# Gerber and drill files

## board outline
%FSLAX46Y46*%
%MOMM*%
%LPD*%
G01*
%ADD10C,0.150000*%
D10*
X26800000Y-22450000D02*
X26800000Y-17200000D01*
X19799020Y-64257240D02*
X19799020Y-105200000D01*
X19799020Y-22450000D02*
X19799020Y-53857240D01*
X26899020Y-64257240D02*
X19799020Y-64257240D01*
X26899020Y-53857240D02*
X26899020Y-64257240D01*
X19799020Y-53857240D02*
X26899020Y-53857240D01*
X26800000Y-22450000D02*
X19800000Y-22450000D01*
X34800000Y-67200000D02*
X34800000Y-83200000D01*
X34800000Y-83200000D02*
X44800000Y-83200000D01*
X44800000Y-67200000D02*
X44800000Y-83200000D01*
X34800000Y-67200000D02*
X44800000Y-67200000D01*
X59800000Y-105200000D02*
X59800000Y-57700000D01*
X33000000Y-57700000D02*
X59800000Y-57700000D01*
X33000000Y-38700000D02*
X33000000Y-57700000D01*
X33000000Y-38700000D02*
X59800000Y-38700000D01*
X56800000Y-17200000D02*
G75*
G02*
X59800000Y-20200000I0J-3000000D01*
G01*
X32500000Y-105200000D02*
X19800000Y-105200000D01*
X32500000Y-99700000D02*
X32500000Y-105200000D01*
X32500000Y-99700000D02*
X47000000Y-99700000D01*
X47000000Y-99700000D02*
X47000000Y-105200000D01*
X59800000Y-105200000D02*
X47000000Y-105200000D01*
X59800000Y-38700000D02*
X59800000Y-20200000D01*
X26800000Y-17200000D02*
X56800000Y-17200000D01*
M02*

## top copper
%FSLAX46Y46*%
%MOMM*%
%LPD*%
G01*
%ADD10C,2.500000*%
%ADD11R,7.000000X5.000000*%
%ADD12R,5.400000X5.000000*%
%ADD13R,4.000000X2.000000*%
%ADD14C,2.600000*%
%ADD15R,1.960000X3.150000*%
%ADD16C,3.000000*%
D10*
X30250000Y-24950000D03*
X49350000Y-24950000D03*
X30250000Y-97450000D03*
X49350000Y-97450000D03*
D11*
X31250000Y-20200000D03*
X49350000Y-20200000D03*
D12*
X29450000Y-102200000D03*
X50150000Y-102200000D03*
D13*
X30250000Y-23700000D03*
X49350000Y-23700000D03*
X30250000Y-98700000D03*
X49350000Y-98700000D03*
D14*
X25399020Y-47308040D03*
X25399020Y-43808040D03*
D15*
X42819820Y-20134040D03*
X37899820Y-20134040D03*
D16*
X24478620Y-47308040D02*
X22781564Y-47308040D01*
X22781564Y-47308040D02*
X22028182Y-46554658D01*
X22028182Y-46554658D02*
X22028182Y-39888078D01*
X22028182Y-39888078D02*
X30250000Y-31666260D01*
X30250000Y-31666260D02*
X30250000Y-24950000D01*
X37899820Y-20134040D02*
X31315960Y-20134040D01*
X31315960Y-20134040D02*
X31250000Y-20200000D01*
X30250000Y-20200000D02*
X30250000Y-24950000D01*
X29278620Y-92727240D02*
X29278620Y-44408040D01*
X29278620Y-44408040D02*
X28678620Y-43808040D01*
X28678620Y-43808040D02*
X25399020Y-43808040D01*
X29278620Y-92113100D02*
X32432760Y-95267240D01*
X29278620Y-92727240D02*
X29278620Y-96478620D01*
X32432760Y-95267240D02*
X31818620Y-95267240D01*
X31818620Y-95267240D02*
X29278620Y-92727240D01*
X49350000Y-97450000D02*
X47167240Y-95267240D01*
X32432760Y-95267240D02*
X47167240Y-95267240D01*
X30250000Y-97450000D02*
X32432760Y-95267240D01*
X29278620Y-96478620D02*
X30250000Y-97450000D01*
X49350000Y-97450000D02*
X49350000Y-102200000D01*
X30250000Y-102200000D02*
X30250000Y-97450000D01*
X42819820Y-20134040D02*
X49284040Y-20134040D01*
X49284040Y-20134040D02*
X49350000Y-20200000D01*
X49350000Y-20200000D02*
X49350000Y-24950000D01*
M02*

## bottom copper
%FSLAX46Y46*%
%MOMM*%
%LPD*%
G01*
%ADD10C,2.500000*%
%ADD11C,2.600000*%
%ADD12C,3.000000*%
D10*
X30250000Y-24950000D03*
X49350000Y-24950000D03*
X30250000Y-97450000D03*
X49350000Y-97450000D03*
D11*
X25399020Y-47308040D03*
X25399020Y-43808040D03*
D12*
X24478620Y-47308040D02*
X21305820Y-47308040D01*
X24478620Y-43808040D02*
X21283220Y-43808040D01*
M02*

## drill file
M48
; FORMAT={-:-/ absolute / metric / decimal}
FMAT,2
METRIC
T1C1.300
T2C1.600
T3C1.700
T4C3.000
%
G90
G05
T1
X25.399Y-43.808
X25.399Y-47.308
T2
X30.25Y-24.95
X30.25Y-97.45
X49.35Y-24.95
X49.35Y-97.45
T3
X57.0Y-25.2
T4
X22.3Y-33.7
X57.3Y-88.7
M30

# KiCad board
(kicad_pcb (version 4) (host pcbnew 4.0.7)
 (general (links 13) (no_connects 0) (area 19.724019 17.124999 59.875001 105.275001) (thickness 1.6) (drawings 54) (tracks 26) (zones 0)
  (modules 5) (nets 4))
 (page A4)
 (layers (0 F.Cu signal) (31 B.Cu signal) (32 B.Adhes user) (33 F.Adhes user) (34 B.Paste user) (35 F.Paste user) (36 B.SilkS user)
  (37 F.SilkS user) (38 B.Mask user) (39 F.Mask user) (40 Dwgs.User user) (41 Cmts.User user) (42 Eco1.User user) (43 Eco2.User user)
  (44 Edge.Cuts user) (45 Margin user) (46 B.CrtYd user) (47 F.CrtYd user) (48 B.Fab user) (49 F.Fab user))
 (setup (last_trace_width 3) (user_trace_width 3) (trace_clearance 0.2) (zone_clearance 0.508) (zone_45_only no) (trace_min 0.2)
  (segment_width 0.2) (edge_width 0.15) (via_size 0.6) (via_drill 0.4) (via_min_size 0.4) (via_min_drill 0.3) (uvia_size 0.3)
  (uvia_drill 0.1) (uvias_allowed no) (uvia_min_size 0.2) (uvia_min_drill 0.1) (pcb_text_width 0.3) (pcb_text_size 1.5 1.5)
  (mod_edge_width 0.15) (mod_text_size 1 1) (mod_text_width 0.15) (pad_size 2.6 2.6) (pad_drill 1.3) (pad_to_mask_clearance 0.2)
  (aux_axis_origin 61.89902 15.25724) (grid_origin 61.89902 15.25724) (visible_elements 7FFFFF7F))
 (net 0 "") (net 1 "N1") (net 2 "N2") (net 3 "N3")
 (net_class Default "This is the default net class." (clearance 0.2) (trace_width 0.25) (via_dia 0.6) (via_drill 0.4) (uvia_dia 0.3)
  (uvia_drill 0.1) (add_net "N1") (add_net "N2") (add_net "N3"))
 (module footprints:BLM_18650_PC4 (layer F.Cu) (at 39.8 61.2)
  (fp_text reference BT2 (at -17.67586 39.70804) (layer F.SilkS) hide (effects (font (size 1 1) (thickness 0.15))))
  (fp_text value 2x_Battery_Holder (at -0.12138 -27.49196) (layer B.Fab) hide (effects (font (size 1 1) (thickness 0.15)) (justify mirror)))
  (pad 1 thru_hole circle (at -9.55 -36.25) (size 2.5 2.5) (drill 1.6) (layers *.Cu *.Mask) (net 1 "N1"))
  (pad 2 thru_hole circle (at 9.55 -36.25) (size 2.5 2.5) (drill 1.6) (layers *.Cu *.Mask) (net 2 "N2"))
  (pad 3 thru_hole circle (at -9.55 36.25) (size 2.5 2.5) (drill 1.6) (layers *.Cu *.Mask) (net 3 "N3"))
  (pad 4 thru_hole circle (at 9.55 36.25) (size 2.5 2.5) (drill 1.6) (layers *.Cu *.Mask) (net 3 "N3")))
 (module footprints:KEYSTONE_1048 (layer F.Cu) (at 39.8 61.2)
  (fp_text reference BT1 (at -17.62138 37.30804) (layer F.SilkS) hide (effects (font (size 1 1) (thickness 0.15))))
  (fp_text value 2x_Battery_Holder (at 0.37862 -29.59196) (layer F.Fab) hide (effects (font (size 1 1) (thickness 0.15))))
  (pad 1 smd rect (at -8.55 -41) (size 7 5) (layers F.Cu F.Paste F.Mask) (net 1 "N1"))
  (pad 2 smd rect (at 9.55 -41) (size 7 5) (layers F.Cu F.Paste F.Mask) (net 2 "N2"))
  (pad 3 smd rect (at -10.35 41) (size 5.4 5) (layers F.Cu F.Paste F.Mask) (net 3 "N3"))
  (pad 4 smd rect (at 10.35 41) (size 5.4 5) (layers F.Cu F.Paste F.Mask) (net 3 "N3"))
  (pad "" np_thru_hole circle (at 17.2 -36) (size 1.7 1.7) (drill 1.7) (layers *.Cu *.Mask))
  (pad "" np_thru_hole circle (at -17.5 -27.5) (size 3 3) (drill 3) (layers *.Cu *.Mask))
  (pad "" np_thru_hole circle (at 17.5 27.5) (size 3 3) (drill 3) (layers *.Cu *.Mask))
  (pad 1 smd rect (at -9.55 -37.5) (size 4 2) (layers F.Cu F.Paste F.Mask) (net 1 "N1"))
  (pad 2 smd rect (at 9.55 -37.5) (size 4 2) (layers F.Cu F.Paste F.Mask) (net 2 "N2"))
  (pad 3 smd rect (at -9.55 37.5) (size 4 2) (layers F.Cu F.Paste F.Mask) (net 3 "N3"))
  (pad 4 smd rect (at 9.55 37.5) (size 4 2) (layers F.Cu F.Paste F.Mask) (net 3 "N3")))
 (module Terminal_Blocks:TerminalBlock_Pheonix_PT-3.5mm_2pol (layer F.Cu) (at 25.39902 43.80804 270)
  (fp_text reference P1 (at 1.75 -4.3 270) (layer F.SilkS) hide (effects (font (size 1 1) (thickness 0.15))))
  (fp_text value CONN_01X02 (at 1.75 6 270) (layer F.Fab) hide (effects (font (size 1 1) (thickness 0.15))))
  (pad 2 thru_hole circle (at 3.5 0 270) (size 2.6 2.6) (drill 1.3) (layers *.Cu *.Mask) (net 1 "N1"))
  (pad 1 thru_hole circle (at 0 0 270) (size 2.6 2.6) (drill 1.3) (layers *.Cu *.Mask) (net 3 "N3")))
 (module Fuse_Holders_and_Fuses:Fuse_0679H (layer F.Cu) (at 40.35982 20.13404)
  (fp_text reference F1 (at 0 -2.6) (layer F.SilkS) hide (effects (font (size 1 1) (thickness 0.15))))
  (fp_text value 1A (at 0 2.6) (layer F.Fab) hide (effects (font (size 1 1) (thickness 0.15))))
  (pad 2 smd rect (at 2.46 0) (size 1.96 3.15) (layers F.Cu F.Paste F.Mask) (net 2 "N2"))
  (pad 1 smd rect (at -2.46 0) (size 1.96 3.15) (layers F.Cu F.Paste F.Mask) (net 1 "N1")))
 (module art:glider (layer F.Cu) (at 30.39902 37.75724)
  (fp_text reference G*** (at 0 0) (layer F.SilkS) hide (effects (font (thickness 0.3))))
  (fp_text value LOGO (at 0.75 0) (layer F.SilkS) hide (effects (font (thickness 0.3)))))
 (gr_line (start 26.8 22.45) (end 26.8 17.2) (layer Edge.Cuts) (width 0.15))
 (gr_line (start 19.79902 64.25724) (end 19.79902 105.2) (layer Edge.Cuts) (width 0.15))
 (gr_line (start 19.79902 22.45) (end 19.79902 53.85724) (layer Edge.Cuts) (width 0.15))
 (gr_line (start 26.89902 64.25724) (end 19.79902 64.25724) (layer Edge.Cuts) (width 0.15))
 (gr_line (start 26.89902 53.85724) (end 26.89902 64.25724) (layer Edge.Cuts) (width 0.15))
 (gr_line (start 19.79902 53.85724) (end 26.89902 53.85724) (layer Edge.Cuts) (width 0.15))
 (gr_line (start 26.8 22.45) (end 19.8 22.45) (layer Edge.Cuts) (width 0.15))
 (gr_line (start 34.8 67.2) (end 34.8 83.2) (layer Edge.Cuts) (width 0.15))
 (gr_line (start 34.8 83.2) (end 44.8 83.2) (layer Edge.Cuts) (width 0.15))
 (gr_line (start 44.8 67.2) (end 44.8 83.2) (layer Edge.Cuts) (width 0.15))
 (gr_line (start 34.8 67.2) (end 44.8 67.2) (layer Edge.Cuts) (width 0.15))
 (gr_line (start 59.8 105.2) (end 59.8 57.7) (layer Edge.Cuts) (width 0.15))
 (gr_line (start 33 57.7) (end 59.8 57.7) (layer Edge.Cuts) (width 0.15))
 (gr_line (start 33 38.7) (end 33 57.7) (layer Edge.Cuts) (width 0.15))
 (gr_line (start 33 38.7) (end 59.8 38.7) (layer Edge.Cuts) (width 0.15))
 (gr_arc (start 56.8 20.2) (end 56.8 17.2) (angle 90) (layer Edge.Cuts) (width 0.15))
 (gr_line (start 32.5 105.2) (end 19.8 105.2) (layer Edge.Cuts) (width 0.15))
 (gr_line (start 32.5 99.7) (end 32.5 105.2) (layer Edge.Cuts) (width 0.15))
 (gr_line (start 32.5 99.7) (end 47 99.7) (layer Edge.Cuts) (width 0.15))
 (gr_line (start 47 99.7) (end 47 105.2) (layer Edge.Cuts) (width 0.15))
 (gr_line (start 59.8 105.2) (end 47 105.2) (layer Edge.Cuts) (width 0.15))
 (gr_line (start 59.8 38.7) (end 59.8 20.2) (layer Edge.Cuts) (width 0.15))
 (gr_line (start 26.8 17.2) (end 56.8 17.2) (layer Edge.Cuts) (width 0.15))
 (segment (start 24.47862 47.30804) (end 22.781564 47.30804) (width 3) (layer F.Cu) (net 1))
 (segment (start 22.781564 47.30804) (end 22.028182 46.554658) (width 3) (layer F.Cu) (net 1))
 (segment (start 22.028182 46.554658) (end 22.028182 39.888078) (width 3) (layer F.Cu) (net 1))
 (segment (start 22.028182 39.888078) (end 30.25 31.66626) (width 3) (layer F.Cu) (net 1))
 (segment (start 30.25 31.66626) (end 30.25 24.95) (width 3) (layer F.Cu) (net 1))
 (segment (start 24.47862 47.30804) (end 21.30582 47.30804) (width 3) (layer B.Cu) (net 1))
 (segment (start 37.89982 20.13404) (end 31.31596 20.13404) (width 3) (layer F.Cu) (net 1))
 (segment (start 31.31596 20.13404) (end 31.25 20.2) (width 3) (layer F.Cu) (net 1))
 (segment (start 30.25 20.2) (end 30.25 24.95) (width 3) (layer F.Cu) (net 1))
 (segment (start 29.27862 92.72724) (end 29.27862 44.40804) (width 3) (layer F.Cu) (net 3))
 (segment (start 29.27862 44.40804) (end 28.67862 43.80804) (width 3) (layer F.Cu) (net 3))
 (segment (start 28.67862 43.80804) (end 25.39902 43.80804) (width 3) (layer F.Cu) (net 3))
 (segment (start 24.47862 43.80804) (end 21.28322 43.80804) (width 3) (layer B.Cu) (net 3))
 (segment (start 29.27862 92.1131) (end 32.43276 95.26724) (width 3) (layer F.Cu) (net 3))
 (segment (start 29.27862 92.72724) (end 29.27862 96.47862) (width 3) (layer F.Cu) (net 3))
 (segment (start 32.43276 95.26724) (end 31.81862 95.26724) (width 3) (layer F.Cu) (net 3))
 (segment (start 31.81862 95.26724) (end 29.27862 92.72724) (width 3) (layer F.Cu) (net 3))
 (segment (start 49.35 97.45) (end 47.16724 95.26724) (width 3) (layer F.Cu) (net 3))
 (segment (start 32.43276 95.26724) (end 47.16724 95.26724) (width 3) (layer F.Cu) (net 3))
 (segment (start 30.25 97.45) (end 32.43276 95.26724) (width 3) (layer F.Cu) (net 3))
 (segment (start 29.27862 96.47862) (end 30.25 97.45) (width 3) (layer F.Cu) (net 3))
 (segment (start 49.35 97.45) (end 49.35 102.2) (width 3) (layer F.Cu) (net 3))
 (segment (start 30.25 102.2) (end 30.25 97.45) (width 3) (layer F.Cu) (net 3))
 (segment (start 42.81982 20.13404) (end 49.28404 20.13404) (width 3) (layer F.Cu) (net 2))
 (segment (start 49.28404 20.13404) (end 49.35 20.2) (width 3) (layer F.Cu) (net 2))
 (segment (start 49.35 20.2) (end 49.35 24.95) (width 3) (layer F.Cu) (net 2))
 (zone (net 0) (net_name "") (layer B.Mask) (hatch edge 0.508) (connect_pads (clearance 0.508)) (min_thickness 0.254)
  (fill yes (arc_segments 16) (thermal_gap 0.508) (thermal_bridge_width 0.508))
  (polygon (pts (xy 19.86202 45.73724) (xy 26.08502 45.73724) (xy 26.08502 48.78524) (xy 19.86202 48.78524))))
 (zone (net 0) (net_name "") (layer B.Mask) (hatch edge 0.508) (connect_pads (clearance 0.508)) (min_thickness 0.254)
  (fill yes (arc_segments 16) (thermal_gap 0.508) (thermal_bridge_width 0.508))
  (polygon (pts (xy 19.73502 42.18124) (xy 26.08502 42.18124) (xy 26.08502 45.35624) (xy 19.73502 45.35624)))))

